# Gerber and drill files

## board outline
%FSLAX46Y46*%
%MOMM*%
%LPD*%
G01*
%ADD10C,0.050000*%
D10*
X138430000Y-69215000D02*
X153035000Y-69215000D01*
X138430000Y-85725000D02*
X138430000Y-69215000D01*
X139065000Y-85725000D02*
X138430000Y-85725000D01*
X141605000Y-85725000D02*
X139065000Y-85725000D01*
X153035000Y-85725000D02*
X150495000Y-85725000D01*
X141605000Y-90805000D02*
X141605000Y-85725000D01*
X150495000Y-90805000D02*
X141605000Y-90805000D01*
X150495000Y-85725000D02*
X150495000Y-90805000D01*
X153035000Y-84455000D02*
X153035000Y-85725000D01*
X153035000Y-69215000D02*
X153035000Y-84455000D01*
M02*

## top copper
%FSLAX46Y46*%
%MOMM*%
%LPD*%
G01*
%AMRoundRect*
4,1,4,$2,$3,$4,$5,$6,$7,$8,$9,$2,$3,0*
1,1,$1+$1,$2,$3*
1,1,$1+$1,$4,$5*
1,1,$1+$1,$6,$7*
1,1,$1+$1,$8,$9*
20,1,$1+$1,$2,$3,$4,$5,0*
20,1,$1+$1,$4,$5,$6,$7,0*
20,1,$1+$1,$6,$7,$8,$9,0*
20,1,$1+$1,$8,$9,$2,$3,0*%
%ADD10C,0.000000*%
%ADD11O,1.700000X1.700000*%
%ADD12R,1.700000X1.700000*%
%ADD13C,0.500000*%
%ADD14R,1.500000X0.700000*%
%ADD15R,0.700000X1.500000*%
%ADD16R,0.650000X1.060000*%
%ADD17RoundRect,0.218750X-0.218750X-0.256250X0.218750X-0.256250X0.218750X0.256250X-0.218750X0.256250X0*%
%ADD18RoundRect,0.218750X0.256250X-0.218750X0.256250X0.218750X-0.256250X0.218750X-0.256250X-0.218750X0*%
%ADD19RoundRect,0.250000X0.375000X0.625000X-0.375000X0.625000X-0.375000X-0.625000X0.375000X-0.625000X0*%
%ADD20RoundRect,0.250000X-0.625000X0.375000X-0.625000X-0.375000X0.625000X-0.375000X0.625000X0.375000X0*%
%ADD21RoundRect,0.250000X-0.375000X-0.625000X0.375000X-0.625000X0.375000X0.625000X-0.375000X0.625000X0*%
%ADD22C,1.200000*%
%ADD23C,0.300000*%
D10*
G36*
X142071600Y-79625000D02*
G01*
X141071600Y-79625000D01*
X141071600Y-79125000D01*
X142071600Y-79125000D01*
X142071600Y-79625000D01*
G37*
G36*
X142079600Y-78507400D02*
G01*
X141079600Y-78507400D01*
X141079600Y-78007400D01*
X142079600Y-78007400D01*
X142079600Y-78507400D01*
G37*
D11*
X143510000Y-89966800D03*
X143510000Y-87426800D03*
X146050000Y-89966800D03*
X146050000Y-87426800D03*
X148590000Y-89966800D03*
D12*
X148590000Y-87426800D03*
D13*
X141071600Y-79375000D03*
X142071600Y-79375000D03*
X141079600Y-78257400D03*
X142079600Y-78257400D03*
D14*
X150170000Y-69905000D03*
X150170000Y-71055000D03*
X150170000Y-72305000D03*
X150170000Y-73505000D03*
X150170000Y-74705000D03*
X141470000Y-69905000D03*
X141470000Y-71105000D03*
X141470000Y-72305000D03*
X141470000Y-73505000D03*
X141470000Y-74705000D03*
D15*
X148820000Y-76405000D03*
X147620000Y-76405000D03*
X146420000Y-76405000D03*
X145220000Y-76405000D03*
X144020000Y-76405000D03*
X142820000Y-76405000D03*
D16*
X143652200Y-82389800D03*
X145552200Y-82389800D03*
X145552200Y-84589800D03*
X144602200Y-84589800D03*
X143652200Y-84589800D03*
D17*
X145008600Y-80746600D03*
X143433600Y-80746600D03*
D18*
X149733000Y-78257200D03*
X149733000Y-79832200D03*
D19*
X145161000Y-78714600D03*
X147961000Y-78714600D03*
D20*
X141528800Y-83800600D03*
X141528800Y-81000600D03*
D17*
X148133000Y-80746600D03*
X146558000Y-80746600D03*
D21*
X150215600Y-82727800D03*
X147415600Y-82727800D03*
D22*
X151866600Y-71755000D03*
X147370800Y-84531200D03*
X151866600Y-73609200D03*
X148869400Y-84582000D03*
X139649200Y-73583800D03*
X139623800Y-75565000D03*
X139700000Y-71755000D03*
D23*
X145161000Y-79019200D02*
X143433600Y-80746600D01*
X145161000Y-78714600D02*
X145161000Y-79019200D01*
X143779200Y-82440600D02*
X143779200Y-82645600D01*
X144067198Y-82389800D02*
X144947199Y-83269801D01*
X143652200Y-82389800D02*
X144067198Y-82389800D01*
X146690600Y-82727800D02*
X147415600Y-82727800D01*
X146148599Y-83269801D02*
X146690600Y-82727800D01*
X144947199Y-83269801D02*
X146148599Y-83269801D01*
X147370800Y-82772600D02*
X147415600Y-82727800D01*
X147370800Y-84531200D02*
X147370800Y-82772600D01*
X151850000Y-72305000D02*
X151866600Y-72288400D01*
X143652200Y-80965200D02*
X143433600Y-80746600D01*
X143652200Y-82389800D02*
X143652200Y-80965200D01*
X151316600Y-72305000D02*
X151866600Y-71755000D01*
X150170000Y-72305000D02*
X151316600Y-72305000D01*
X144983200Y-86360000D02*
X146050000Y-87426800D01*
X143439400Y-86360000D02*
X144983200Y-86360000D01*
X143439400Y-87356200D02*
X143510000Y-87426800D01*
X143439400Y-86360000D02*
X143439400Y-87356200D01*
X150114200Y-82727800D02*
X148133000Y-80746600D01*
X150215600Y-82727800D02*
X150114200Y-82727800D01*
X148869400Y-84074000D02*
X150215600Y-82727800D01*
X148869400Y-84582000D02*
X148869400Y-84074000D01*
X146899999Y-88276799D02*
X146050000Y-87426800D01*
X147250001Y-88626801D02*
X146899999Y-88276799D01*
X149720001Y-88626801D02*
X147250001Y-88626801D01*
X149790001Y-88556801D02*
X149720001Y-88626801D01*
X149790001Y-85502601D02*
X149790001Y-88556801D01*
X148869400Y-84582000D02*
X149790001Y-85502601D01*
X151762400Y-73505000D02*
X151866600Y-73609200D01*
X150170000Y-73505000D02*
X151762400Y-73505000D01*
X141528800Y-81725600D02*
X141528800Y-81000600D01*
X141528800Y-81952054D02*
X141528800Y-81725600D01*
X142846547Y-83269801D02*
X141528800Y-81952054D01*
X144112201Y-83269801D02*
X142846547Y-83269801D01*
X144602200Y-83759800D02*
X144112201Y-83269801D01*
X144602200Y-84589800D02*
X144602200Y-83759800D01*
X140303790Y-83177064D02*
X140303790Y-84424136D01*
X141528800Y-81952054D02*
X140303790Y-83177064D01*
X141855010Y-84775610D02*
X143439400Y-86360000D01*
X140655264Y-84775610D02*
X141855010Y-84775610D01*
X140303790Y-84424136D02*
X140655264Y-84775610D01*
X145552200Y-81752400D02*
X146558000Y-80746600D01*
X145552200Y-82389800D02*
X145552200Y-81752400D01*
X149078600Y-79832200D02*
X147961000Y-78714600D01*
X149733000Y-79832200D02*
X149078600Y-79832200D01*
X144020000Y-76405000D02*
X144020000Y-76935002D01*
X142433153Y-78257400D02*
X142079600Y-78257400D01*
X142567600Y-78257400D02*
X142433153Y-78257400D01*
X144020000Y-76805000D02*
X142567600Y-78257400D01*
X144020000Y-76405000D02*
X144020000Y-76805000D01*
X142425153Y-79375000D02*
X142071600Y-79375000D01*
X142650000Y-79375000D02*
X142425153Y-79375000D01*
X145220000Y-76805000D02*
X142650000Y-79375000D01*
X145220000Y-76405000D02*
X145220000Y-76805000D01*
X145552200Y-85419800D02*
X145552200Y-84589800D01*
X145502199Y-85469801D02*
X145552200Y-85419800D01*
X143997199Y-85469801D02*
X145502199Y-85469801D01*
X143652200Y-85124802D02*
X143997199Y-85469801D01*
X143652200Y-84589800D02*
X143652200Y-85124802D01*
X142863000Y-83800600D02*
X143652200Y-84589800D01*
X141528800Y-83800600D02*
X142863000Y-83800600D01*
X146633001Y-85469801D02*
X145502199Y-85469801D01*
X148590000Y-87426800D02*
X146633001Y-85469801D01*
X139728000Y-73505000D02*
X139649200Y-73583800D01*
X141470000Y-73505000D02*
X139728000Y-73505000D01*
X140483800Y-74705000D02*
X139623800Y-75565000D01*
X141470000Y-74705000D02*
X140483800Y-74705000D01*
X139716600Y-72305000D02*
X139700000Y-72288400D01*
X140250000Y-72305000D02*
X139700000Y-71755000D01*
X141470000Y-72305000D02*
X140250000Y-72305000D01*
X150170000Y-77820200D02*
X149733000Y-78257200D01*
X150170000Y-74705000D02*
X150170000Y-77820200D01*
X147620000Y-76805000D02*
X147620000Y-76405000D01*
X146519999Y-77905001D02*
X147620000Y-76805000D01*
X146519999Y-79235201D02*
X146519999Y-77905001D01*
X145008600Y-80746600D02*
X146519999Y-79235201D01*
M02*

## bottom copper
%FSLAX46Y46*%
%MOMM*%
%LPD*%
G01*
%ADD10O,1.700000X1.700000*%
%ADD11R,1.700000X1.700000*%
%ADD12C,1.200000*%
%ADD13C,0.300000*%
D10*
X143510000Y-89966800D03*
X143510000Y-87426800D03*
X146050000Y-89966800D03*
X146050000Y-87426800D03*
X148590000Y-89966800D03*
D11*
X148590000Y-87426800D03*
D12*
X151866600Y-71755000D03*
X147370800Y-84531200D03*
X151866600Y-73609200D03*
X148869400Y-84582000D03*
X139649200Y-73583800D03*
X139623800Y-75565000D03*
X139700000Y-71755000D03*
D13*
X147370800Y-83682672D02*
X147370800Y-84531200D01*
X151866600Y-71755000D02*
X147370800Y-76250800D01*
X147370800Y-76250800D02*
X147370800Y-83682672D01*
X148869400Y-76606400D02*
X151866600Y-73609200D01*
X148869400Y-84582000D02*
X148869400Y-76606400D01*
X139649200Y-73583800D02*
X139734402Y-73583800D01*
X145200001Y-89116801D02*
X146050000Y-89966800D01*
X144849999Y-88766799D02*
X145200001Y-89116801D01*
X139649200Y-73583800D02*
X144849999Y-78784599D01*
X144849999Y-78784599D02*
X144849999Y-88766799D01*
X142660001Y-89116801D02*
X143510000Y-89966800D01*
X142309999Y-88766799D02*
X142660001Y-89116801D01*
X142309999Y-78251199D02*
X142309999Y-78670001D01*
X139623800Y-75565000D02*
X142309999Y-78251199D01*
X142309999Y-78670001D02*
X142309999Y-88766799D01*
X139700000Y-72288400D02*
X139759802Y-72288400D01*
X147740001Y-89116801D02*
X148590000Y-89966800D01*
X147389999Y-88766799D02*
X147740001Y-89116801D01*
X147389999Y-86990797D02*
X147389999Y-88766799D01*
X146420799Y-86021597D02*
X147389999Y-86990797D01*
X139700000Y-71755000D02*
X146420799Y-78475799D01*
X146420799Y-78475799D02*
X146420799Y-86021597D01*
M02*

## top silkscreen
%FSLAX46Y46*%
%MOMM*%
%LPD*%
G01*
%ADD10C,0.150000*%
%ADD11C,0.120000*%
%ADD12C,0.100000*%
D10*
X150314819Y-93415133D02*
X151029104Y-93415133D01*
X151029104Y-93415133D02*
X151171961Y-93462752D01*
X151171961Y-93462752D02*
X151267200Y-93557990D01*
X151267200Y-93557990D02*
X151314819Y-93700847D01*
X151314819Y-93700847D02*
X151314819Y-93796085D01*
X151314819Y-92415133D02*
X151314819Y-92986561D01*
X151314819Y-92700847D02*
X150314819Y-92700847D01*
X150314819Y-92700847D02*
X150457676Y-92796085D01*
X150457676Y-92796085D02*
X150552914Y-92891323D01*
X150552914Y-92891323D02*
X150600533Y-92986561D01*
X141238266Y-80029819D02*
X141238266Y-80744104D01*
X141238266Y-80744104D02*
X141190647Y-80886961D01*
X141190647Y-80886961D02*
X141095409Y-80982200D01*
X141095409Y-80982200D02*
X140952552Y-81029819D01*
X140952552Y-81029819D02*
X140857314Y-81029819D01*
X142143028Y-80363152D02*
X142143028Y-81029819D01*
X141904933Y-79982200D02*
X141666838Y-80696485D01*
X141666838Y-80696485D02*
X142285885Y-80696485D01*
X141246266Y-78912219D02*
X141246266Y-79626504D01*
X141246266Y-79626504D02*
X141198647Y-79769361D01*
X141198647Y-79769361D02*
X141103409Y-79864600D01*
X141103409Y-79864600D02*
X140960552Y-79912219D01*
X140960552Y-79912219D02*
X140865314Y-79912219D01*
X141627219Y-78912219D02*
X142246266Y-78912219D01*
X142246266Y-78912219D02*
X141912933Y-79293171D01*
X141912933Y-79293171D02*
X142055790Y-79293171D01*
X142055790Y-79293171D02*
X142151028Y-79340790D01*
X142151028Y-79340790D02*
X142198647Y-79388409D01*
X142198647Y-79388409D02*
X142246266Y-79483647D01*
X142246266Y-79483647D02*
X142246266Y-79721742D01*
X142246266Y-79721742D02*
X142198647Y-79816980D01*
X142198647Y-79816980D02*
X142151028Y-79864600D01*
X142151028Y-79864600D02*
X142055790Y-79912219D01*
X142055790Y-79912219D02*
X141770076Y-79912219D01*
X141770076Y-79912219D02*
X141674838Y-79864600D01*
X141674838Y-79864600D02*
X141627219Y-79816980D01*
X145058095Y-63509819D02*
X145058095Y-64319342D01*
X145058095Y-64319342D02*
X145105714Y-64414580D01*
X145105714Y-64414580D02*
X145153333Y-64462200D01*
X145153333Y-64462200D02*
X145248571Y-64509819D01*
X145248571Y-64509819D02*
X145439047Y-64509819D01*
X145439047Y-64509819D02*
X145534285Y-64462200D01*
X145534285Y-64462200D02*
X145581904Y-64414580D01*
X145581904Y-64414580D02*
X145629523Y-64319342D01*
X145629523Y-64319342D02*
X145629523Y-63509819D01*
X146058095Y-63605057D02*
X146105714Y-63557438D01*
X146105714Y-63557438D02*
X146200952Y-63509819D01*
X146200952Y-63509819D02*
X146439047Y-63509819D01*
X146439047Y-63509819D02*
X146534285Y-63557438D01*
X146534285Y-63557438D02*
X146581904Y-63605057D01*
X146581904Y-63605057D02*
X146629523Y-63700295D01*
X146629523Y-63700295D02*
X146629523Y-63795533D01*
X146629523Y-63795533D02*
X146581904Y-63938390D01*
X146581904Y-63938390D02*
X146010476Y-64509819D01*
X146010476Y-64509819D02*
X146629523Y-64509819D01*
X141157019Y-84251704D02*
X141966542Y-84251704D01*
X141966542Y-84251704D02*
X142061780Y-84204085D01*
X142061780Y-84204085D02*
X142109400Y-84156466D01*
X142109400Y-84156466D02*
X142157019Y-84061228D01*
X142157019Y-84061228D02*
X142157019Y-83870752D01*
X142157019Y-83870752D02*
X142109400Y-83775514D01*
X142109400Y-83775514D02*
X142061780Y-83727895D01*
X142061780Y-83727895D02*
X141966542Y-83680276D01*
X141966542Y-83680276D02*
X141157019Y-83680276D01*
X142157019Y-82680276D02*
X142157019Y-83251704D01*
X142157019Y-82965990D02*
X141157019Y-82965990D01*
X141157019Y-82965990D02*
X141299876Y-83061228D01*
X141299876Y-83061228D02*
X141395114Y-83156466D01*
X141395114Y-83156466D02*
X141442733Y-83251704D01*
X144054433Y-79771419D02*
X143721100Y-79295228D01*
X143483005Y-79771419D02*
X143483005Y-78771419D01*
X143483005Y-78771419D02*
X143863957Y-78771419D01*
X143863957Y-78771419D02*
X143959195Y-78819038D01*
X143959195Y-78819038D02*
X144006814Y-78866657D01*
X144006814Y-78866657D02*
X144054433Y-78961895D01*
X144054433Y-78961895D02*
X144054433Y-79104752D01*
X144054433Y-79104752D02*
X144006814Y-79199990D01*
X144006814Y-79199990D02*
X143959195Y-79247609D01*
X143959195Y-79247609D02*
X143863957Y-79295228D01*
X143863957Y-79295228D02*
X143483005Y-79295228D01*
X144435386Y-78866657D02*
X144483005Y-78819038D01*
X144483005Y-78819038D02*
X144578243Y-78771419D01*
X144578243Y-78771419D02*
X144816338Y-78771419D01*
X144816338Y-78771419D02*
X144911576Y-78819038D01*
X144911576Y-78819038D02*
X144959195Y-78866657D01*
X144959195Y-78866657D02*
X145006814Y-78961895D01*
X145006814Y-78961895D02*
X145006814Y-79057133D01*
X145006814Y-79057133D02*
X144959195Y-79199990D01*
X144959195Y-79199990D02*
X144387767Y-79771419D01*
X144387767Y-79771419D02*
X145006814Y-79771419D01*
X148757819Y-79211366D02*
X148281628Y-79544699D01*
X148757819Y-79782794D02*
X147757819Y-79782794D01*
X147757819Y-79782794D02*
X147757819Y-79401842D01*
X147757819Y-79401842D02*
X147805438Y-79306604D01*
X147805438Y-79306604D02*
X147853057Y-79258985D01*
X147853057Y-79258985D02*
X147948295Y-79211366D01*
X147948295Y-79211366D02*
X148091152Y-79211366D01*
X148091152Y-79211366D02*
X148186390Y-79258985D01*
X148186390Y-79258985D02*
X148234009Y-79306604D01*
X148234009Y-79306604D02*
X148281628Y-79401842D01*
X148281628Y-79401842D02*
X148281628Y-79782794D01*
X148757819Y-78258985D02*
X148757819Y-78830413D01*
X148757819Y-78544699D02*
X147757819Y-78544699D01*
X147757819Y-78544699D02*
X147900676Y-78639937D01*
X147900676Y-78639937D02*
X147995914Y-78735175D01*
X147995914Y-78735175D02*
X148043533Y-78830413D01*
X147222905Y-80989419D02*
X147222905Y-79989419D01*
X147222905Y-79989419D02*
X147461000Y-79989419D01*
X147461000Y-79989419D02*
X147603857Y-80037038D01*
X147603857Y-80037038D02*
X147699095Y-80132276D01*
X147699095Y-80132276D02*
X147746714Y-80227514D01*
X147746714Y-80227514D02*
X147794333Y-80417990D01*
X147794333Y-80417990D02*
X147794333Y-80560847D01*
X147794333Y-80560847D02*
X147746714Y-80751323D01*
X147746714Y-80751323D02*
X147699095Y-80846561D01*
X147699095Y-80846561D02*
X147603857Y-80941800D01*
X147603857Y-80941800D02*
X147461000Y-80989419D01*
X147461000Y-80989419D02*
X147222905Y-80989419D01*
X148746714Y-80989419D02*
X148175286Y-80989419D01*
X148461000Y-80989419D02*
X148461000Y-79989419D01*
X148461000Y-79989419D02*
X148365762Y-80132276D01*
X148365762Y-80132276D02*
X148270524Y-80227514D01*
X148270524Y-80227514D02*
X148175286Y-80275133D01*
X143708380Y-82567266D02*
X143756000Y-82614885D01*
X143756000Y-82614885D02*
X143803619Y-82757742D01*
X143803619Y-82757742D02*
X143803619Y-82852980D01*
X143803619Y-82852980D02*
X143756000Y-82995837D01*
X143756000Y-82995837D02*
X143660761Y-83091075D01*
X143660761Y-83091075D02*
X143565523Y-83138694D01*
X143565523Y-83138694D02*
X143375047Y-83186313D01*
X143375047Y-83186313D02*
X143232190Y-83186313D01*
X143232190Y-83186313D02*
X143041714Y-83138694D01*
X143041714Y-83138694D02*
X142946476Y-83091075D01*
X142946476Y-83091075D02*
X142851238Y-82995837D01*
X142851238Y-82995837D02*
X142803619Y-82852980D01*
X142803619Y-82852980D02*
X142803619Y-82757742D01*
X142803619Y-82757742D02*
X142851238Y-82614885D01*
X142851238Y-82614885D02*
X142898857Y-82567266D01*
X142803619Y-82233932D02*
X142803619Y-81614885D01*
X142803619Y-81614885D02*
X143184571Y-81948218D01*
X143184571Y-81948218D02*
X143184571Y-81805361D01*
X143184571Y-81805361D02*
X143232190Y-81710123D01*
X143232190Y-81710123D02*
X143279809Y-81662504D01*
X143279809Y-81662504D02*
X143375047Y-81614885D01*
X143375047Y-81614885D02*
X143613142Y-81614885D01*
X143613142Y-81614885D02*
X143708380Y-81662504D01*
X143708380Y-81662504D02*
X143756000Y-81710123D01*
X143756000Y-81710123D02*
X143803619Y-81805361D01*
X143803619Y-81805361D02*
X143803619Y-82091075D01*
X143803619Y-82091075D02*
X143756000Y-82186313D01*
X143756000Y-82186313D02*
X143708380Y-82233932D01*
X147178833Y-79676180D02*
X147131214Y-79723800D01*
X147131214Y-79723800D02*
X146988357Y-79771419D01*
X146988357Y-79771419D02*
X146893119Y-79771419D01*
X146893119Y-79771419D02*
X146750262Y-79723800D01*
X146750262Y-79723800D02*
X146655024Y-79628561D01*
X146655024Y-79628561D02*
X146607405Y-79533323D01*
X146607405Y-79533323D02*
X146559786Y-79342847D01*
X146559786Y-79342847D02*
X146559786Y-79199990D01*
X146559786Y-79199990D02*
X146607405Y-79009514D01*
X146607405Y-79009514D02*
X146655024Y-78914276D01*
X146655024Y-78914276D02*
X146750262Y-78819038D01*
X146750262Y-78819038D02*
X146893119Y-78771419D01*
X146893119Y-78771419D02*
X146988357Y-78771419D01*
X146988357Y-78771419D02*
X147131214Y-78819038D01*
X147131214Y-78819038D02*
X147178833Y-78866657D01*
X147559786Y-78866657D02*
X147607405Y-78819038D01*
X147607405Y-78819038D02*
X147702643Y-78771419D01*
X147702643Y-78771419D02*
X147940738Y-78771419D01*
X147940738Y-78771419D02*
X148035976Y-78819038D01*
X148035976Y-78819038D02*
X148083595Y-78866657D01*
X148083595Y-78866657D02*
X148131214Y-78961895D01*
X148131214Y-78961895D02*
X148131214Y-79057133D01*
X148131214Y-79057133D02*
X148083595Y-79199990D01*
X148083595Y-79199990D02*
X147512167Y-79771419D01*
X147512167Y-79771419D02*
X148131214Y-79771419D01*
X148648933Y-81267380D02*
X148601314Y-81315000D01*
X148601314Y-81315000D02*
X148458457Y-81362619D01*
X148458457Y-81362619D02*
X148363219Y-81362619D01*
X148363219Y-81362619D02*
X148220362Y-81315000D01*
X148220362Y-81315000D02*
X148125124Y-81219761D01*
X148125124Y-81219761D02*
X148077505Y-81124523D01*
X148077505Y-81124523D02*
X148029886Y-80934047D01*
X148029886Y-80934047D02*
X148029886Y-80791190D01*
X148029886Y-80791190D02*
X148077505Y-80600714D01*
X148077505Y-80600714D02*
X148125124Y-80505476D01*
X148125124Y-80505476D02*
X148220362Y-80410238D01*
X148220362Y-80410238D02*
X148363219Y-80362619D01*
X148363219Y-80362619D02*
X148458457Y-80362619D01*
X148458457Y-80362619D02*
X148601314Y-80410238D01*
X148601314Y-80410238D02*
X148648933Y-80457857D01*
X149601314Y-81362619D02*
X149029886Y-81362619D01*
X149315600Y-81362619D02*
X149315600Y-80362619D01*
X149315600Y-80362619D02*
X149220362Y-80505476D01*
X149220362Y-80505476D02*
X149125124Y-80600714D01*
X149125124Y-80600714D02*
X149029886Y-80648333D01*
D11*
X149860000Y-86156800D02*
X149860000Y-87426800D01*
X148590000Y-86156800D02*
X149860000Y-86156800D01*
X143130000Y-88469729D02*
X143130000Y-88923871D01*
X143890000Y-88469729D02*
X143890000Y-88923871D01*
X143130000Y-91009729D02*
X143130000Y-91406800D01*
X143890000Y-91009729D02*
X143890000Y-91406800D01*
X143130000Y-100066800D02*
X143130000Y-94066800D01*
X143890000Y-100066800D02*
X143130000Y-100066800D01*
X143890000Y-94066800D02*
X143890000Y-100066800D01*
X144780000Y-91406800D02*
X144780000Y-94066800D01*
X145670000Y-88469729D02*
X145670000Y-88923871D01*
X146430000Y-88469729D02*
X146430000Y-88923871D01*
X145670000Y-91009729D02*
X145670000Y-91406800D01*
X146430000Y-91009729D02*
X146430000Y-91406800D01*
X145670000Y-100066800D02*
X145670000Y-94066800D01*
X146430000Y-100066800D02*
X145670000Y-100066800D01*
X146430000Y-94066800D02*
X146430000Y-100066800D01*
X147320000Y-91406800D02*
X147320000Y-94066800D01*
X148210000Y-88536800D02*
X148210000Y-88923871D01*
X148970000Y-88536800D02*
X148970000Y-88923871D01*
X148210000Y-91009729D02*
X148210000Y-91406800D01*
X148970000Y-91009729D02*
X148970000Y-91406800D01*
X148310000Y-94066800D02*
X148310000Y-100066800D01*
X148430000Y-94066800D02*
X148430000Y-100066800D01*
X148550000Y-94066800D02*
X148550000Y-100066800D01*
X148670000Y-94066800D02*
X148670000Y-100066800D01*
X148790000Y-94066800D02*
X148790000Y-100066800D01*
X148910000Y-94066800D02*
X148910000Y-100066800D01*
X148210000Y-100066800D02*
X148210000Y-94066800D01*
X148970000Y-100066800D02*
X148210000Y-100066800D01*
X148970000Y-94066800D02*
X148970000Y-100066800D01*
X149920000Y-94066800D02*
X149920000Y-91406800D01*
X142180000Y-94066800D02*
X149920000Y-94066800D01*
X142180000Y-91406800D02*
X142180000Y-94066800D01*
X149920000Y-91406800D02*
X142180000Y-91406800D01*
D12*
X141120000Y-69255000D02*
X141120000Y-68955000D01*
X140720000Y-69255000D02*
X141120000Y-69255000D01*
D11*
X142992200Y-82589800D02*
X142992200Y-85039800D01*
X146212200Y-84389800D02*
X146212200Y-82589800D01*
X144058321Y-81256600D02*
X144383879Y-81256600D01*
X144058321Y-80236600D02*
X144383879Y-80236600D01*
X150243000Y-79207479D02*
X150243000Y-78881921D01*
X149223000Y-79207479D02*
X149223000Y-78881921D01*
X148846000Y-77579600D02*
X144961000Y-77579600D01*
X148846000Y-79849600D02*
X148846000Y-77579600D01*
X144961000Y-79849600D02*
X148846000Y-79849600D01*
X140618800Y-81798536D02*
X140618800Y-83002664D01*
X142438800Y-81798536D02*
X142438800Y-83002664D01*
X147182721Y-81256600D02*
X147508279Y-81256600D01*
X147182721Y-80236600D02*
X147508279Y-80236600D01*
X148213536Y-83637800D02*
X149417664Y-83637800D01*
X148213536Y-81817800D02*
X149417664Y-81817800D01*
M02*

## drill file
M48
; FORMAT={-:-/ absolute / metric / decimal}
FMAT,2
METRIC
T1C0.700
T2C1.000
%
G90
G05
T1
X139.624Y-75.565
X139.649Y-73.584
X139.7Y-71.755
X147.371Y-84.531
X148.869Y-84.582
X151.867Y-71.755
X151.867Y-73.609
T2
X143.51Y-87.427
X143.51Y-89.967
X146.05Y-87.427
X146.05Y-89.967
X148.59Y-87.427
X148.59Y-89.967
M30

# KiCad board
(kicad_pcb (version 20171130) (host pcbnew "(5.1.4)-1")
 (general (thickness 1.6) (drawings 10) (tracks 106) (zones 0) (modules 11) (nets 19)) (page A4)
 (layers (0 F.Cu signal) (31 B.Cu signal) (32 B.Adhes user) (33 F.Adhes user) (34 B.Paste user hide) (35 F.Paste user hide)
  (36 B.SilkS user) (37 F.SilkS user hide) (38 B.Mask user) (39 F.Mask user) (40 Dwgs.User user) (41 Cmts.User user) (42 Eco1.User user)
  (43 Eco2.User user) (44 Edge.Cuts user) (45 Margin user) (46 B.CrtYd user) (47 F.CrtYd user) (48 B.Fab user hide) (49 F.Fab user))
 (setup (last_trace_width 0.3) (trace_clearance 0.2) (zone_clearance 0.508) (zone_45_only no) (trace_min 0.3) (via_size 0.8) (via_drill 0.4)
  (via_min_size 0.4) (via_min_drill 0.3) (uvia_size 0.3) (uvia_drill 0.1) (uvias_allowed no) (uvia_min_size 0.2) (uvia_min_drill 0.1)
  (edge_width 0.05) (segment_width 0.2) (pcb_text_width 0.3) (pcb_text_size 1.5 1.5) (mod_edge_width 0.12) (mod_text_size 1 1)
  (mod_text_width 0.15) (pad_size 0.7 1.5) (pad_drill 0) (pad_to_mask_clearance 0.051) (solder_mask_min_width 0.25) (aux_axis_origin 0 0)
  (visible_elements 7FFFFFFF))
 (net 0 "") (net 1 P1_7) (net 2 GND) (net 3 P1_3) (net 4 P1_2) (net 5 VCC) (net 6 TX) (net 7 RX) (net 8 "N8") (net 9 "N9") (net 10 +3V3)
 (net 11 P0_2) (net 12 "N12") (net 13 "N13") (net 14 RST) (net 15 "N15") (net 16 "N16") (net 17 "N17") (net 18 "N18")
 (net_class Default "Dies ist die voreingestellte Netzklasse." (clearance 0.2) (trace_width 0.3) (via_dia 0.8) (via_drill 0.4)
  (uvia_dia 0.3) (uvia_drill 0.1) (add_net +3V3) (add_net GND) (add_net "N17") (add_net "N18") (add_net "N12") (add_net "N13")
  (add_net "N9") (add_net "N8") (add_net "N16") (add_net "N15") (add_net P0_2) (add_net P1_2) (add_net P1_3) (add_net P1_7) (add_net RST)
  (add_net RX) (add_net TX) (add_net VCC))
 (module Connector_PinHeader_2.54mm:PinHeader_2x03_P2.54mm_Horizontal (layer F.Cu) (at 148.59 87.4268 270)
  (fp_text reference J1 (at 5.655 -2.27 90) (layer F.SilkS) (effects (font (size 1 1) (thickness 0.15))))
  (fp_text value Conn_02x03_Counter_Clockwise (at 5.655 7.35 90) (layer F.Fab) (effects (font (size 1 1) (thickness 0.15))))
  (fp_line (start -1.27 -1.27) (end 0 -1.27) (layer F.SilkS) (width 0.12))
  (fp_line (start -1.27 0) (end -1.27 -1.27) (layer F.SilkS) (width 0.12))
  (fp_line (start 1.042929 5.46) (end 1.497071 5.46) (layer F.SilkS) (width 0.12))
  (fp_line (start 1.042929 4.7) (end 1.497071 4.7) (layer F.SilkS) (width 0.12))
  (fp_line (start 3.582929 5.46) (end 3.98 5.46) (layer F.SilkS) (width 0.12))
  (fp_line (start 3.582929 4.7) (end 3.98 4.7) (layer F.SilkS) (width 0.12))
  (fp_line (start 12.64 5.46) (end 6.64 5.46) (layer F.SilkS) (width 0.12))
  (fp_line (start 12.64 4.7) (end 12.64 5.46) (layer F.SilkS) (width 0.12))
  (fp_line (start 6.64 4.7) (end 12.64 4.7) (layer F.SilkS) (width 0.12))
  (fp_line (start 3.98 3.81) (end 6.64 3.81) (layer F.SilkS) (width 0.12))
  (fp_line (start 1.042929 2.92) (end 1.497071 2.92) (layer F.SilkS) (width 0.12))
  (fp_line (start 1.042929 2.16) (end 1.497071 2.16) (layer F.SilkS) (width 0.12))
  (fp_line (start 3.582929 2.92) (end 3.98 2.92) (layer F.SilkS) (width 0.12))
  (fp_line (start 3.582929 2.16) (end 3.98 2.16) (layer F.SilkS) (width 0.12))
  (fp_line (start 12.64 2.92) (end 6.64 2.92) (layer F.SilkS) (width 0.12))
  (fp_line (start 12.64 2.16) (end 12.64 2.92) (layer F.SilkS) (width 0.12))
  (fp_line (start 6.64 2.16) (end 12.64 2.16) (layer F.SilkS) (width 0.12))
  (fp_line (start 3.98 1.27) (end 6.64 1.27) (layer F.SilkS) (width 0.12))
  (fp_line (start 1.11 0.38) (end 1.497071 0.38) (layer F.SilkS) (width 0.12))
  (fp_line (start 1.11 -0.38) (end 1.497071 -0.38) (layer F.SilkS) (width 0.12))
  (fp_line (start 3.582929 0.38) (end 3.98 0.38) (layer F.SilkS) (width 0.12))
  (fp_line (start 3.582929 -0.38) (end 3.98 -0.38) (layer F.SilkS) (width 0.12))
  (fp_line (start 6.64 0.28) (end 12.64 0.28) (layer F.SilkS) (width 0.12))
  (fp_line (start 6.64 0.16) (end 12.64 0.16) (layer F.SilkS) (width 0.12))
  (fp_line (start 6.64 0.04) (end 12.64 0.04) (layer F.SilkS) (width 0.12))
  (fp_line (start 6.64 -0.08) (end 12.64 -0.08) (layer F.SilkS) (width 0.12))
  (fp_line (start 6.64 -0.2) (end 12.64 -0.2) (layer F.SilkS) (width 0.12))
  (fp_line (start 6.64 -0.32) (end 12.64 -0.32) (layer F.SilkS) (width 0.12))
  (fp_line (start 12.64 0.38) (end 6.64 0.38) (layer F.SilkS) (width 0.12))
  (fp_line (start 12.64 -0.38) (end 12.64 0.38) (layer F.SilkS) (width 0.12))
  (fp_line (start 6.64 -0.38) (end 12.64 -0.38) (layer F.SilkS) (width 0.12))
  (fp_line (start 6.64 -1.33) (end 3.98 -1.33) (layer F.SilkS) (width 0.12))
  (fp_line (start 6.64 6.41) (end 6.64 -1.33) (layer F.SilkS) (width 0.12))
  (fp_line (start 3.98 6.41) (end 6.64 6.41) (layer F.SilkS) (width 0.12))
  (fp_line (start 3.98 -1.33) (end 3.98 6.41) (layer F.SilkS) (width 0.12))
  (pad 6 thru_hole oval (at 2.54 5.08 270) (size 1.7 1.7) (drill 1) (layers *.Cu) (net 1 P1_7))
  (pad 5 thru_hole oval (at 0 5.08 270) (size 1.7 1.7) (drill 1) (layers *.Cu) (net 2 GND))
  (pad 4 thru_hole oval (at 2.54 2.54 270) (size 1.7 1.7) (drill 1) (layers *.Cu) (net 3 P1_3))
  (pad 3 thru_hole oval (at 0 2.54 270) (size 1.7 1.7) (drill 1) (layers *.Cu) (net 2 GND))
  (pad 2 thru_hole oval (at 2.54 0 270) (size 1.7 1.7) (drill 1) (layers *.Cu) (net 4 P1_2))
  (pad 1 thru_hole rect (at 0 0 270) (size 1.7 1.7) (drill 1) (layers *.Cu) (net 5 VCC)))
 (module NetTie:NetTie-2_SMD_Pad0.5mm (layer F.Cu) (at 141.5716 79.375 180)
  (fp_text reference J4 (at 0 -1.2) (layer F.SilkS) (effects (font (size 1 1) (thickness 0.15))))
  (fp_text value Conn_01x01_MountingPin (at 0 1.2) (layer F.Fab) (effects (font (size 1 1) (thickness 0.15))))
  (fp_poly (pts (xy -0.5 -0.25) (xy 0.5 -0.25) (xy 0.5 0.25) (xy -0.5 0.25)) (layer F.Cu) (width 0))
  (pad 2 smd circle (at 0.5 0 180) (size 0.5 0.5) (layers F.Cu))
  (pad 1 smd circle (at -0.5 0 180) (size 0.5 0.5) (layers F.Cu) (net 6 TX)))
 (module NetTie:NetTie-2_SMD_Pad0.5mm (layer F.Cu) (at 141.5796 78.2574 180)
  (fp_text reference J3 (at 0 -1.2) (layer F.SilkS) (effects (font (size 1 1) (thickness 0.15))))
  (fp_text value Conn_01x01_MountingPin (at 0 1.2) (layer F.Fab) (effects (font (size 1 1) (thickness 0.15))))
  (fp_poly (pts (xy -0.5 -0.25) (xy 0.5 -0.25) (xy 0.5 0.25) (xy -0.5 0.25)) (layer F.Cu) (width 0))
  (pad 2 smd circle (at 0.5 0 180) (size 0.5 0.5) (layers F.Cu))
  (pad 1 smd circle (at -0.5 0 180) (size 0.5 0.5) (layers F.Cu) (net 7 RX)))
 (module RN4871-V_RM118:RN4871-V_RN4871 (layer F.Cu) (at 145.82 73.355)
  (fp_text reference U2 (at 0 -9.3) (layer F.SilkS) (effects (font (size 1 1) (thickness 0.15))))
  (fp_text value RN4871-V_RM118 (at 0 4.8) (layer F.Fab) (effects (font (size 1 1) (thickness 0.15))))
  (fp_line (start -4.7 -4.1) (end -4.7 -4.4) (layer F.SilkS) (width 0.1))
  (fp_line (start -5.1 -4.1) (end -4.7 -4.1) (layer F.SilkS) (width 0.1))
  (pad 16 smd rect (at 4.35 -3.45 90) (size 0.7 1.5) (layers F.Cu) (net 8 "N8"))
  (pad 15 smd rect (at 4.35 -2.3 90) (size 0.7 1.5) (layers F.Cu) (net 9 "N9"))
  (pad 14 smd rect (at 4.35 -1.05 90) (size 0.7 1.5) (layers F.Cu F.Paste F.Mask) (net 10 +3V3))
  (pad 13 smd rect (at 4.35 0.15 90) (size 0.7 1.5) (layers F.Cu F.Paste F.Mask) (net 2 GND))
  (pad 12 smd rect (at 4.35 1.35 90) (size 0.7 1.5) (layers F.Cu F.Paste F.Mask) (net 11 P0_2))
  (pad 1 smd rect (at -4.35 -3.45 90) (size 0.7 1.5) (layers F.Cu) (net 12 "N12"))
  (pad 2 smd rect (at -4.35 -2.25 90) (size 0.7 1.5) (layers F.Cu) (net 2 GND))
  (pad 3 smd rect (at -4.35 -1.05 90) (size 0.7 1.5) (layers F.Cu F.Paste F.Mask) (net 4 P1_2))
  (pad 4 smd rect (at -4.35 0.15 90) (size 0.7 1.5) (layers F.Cu F.Paste F.Mask) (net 3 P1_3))
  (pad 5 smd rect (at -4.35 1.35 90) (size 0.7 1.5) (layers F.Cu F.Paste F.Mask) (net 1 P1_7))
  (pad 11 smd rect (at 3 3.05) (size 0.7 1.5) (layers F.Cu) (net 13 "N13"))
  (pad 10 smd rect (at 1.8 3.05) (size 0.7 1.5) (layers F.Cu F.Paste F.Mask) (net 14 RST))
  (pad 9 smd rect (at 0.6 3.05) (size 0.7 1.5) (layers F.Cu) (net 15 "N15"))
  (pad 8 smd rect (at -0.6 3.05) (size 0.7 1.5) (layers F.Cu F.Paste F.Mask) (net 6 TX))
  (pad 7 smd rect (at -1.8 3.05) (size 0.7 1.5) (layers F.Cu F.Paste F.Mask) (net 7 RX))
  (pad 6 smd rect (at -3 3.05) (size 0.7 1.5) (layers F.Cu) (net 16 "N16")))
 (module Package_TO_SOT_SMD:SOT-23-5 (layer F.Cu) (at 144.6022 83.4898 90)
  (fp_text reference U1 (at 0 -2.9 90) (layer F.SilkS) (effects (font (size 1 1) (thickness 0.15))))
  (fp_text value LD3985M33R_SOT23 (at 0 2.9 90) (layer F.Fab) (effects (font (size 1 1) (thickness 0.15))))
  (fp_line (start 0.9 -1.61) (end -1.55 -1.61) (layer F.SilkS) (width 0.12))
  (fp_line (start -0.9 1.61) (end 0.9 1.61) (layer F.SilkS) (width 0.12))
  (pad 5 smd rect (at 1.1 -0.95 90) (size 1.06 0.65) (layers F.Cu F.Paste F.Mask) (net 10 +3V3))
  (pad 4 smd rect (at 1.1 0.95 90) (size 1.06 0.65) (layers F.Cu F.Paste F.Mask) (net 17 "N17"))
  (pad 3 smd rect (at -1.1 0.95 90) (size 1.06 0.65) (layers F.Cu F.Paste F.Mask) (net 5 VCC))
  (pad 2 smd rect (at -1.1 0 90) (size 1.06 0.65) (layers F.Cu F.Paste F.Mask) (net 2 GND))
  (pad 1 smd rect (at -1.1 -0.95 90) (size 1.06 0.65) (layers F.Cu F.Paste F.Mask) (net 5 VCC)))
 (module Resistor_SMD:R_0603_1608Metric (layer F.Cu) (at 144.2211 80.7466)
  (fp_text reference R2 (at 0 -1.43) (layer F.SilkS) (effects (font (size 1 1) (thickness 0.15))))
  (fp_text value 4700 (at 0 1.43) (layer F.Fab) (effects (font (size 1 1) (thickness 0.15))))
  (fp_line (start -0.162779 0.51) (end 0.162779 0.51) (layer F.SilkS) (width 0.12))
  (fp_line (start -0.162779 -0.51) (end 0.162779 -0.51) (layer F.SilkS) (width 0.12))
  (pad 2 smd roundrect (at 0.7875 0) (size 0.875 0.95) (layers F.Cu F.Paste F.Mask) (roundrect_rratio 0.25) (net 14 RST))
  (pad 1 smd roundrect (at -0.7875 0) (size 0.875 0.95) (layers F.Cu F.Paste F.Mask) (roundrect_rratio 0.25) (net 10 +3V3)))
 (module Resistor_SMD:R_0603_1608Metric (layer F.Cu) (at 149.733 79.0447 90)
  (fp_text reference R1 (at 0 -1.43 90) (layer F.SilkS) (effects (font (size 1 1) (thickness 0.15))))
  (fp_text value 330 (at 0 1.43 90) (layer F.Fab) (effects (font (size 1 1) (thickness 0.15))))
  (fp_line (start -0.162779 0.51) (end 0.162779 0.51) (layer F.SilkS) (width 0.12))
  (fp_line (start -0.162779 -0.51) (end 0.162779 -0.51) (layer F.SilkS) (width 0.12))
  (pad 2 smd roundrect (at 0.7875 0 90) (size 0.875 0.95) (layers F.Cu F.Paste F.Mask) (roundrect_rratio 0.25) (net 11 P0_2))
  (pad 1 smd roundrect (at -0.7875 0 90) (size 0.875 0.95) (layers F.Cu F.Paste F.Mask) (roundrect_rratio 0.25) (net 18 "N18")))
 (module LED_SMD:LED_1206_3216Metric (layer F.Cu) (at 146.561 78.7146 180)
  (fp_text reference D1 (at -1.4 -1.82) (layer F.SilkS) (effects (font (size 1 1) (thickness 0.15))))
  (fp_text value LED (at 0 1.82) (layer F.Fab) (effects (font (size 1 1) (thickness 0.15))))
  (fp_line (start -2.285 1.135) (end 1.6 1.135) (layer F.SilkS) (width 0.12))
  (fp_line (start -2.285 -1.135) (end -2.285 1.135) (layer F.SilkS) (width 0.12))
  (fp_line (start 1.6 -1.135) (end -2.285 -1.135) (layer F.SilkS) (width 0.12))
  (pad 2 smd roundrect (at 1.4 0 180) (size 1.25 1.75) (layers F.Cu F.Paste F.Mask) (roundrect_rratio 0.2) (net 10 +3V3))
  (pad 1 smd roundrect (at -1.4 0 180) (size 1.25 1.75) (layers F.Cu F.Paste F.Mask) (roundrect_rratio 0.2) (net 18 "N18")))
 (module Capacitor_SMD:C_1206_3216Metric (layer F.Cu) (at 141.5288 82.4006 270)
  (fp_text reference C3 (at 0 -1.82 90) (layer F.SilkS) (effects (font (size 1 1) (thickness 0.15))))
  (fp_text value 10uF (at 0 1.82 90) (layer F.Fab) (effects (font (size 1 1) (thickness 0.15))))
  (fp_line (start -0.602064 0.91) (end 0.602064 0.91) (layer F.SilkS) (width 0.12))
  (fp_line (start -0.602064 -0.91) (end 0.602064 -0.91) (layer F.SilkS) (width 0.12))
  (pad 2 smd roundrect (at 1.4 0 270) (size 1.25 1.75) (layers F.Cu F.Paste F.Mask) (roundrect_rratio 0.2) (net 5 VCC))
  (pad 1 smd roundrect (at -1.4 0 270) (size 1.25 1.75) (layers F.Cu F.Paste F.Mask) (roundrect_rratio 0.2) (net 2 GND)))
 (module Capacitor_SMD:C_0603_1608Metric (layer F.Cu) (at 147.3455 80.7466)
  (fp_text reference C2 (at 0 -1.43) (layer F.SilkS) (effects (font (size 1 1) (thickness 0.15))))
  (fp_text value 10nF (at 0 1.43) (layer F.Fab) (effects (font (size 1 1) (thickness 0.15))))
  (fp_line (start -0.162779 0.51) (end 0.162779 0.51) (layer F.SilkS) (width 0.12))
  (fp_line (start -0.162779 -0.51) (end 0.162779 -0.51) (layer F.SilkS) (width 0.12))
  (pad 2 smd roundrect (at 0.7875 0) (size 0.875 0.95) (layers F.Cu F.Paste F.Mask) (roundrect_rratio 0.25) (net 2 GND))
  (pad 1 smd roundrect (at -0.7875 0) (size 0.875 0.95) (layers F.Cu F.Paste F.Mask) (roundrect_rratio 0.25) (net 17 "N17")))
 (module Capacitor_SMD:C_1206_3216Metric (layer F.Cu) (at 148.8156 82.7278)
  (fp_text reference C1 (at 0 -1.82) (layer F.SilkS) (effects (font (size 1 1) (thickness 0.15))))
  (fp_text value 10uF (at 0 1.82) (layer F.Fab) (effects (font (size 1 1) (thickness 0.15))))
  (fp_line (start -0.602064 0.91) (end 0.602064 0.91) (layer F.SilkS) (width 0.12))
  (fp_line (start -0.602064 -0.91) (end 0.602064 -0.91) (layer F.SilkS) (width 0.12))
  (pad 2 smd roundrect (at 1.4 0) (size 1.25 1.75) (layers F.Cu F.Paste F.Mask) (roundrect_rratio 0.2) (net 2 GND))
  (pad 1 smd roundrect (at -1.4 0) (size 1.25 1.75) (layers F.Cu F.Paste F.Mask) (roundrect_rratio 0.2) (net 10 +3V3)))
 (gr_line (start 138.43 69.215) (end 153.035 69.215) (layer Edge.Cuts) (width 0.05))
 (gr_line (start 138.43 85.725) (end 138.43 69.215) (layer Edge.Cuts) (width 0.05))
 (gr_line (start 139.065 85.725) (end 138.43 85.725) (layer Edge.Cuts) (width 0.05))
 (gr_line (start 141.605 85.725) (end 139.065 85.725) (layer Edge.Cuts) (width 0.05))
 (gr_line (start 153.035 85.725) (end 150.495 85.725) (layer Edge.Cuts) (width 0.05))
 (gr_line (start 141.605 90.805) (end 141.605 85.725) (layer Edge.Cuts) (width 0.05))
 (gr_line (start 150.495 90.805) (end 141.605 90.805) (layer Edge.Cuts) (width 0.05))
 (gr_line (start 150.495 85.725) (end 150.495 90.805) (layer Edge.Cuts) (width 0.05))
 (gr_line (start 153.035 84.455) (end 153.035 85.725) (layer Edge.Cuts) (width 0.05))
 (gr_line (start 153.035 69.215) (end 153.035 84.455) (layer Edge.Cuts) (width 0.05))
 (via (at 151.8666 71.755) (size 1.2) (drill 0.7) (layers F.Cu B.Cu) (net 10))
 (via (at 147.3708 84.5312) (size 1.2) (drill 0.7) (layers F.Cu B.Cu) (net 10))
 (segment (start 145.161 79.0192) (end 143.4336 80.7466) (width 0.3) (layer F.Cu) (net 10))
 (segment (start 145.161 78.7146) (end 145.161 79.0192) (width 0.3) (layer F.Cu) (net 10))
 (segment (start 143.7792 82.4406) (end 143.7792 82.6456) (width 0.3) (layer F.Cu) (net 10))
 (segment (start 144.067198 82.3898) (end 144.947199 83.269801) (width 0.3) (layer F.Cu) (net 10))
 (segment (start 143.6522 82.3898) (end 144.067198 82.3898) (width 0.3) (layer F.Cu) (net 10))
 (segment (start 146.6906 82.7278) (end 147.4156 82.7278) (width 0.3) (layer F.Cu) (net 10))
 (segment (start 146.148599 83.269801) (end 146.6906 82.7278) (width 0.3) (layer F.Cu) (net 10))
 (segment (start 144.947199 83.269801) (end 146.148599 83.269801) (width 0.3) (layer F.Cu) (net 10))
 (segment (start 147.3708 82.7726) (end 147.4156 82.7278) (width 0.3) (layer F.Cu) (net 10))
 (segment (start 147.3708 84.5312) (end 147.3708 82.7726) (width 0.3) (layer F.Cu) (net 10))
 (segment (start 151.85 72.305) (end 151.8666 72.2884) (width 0.3) (layer F.Cu) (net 10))
 (segment (start 147.3708 83.682672) (end 147.3708 84.5312) (width 0.3) (layer B.Cu) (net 10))
 (segment (start 143.6522 80.9652) (end 143.4336 80.7466) (width 0.3) (layer F.Cu) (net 10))
 (segment (start 143.6522 82.3898) (end 143.6522 80.9652) (width 0.3) (layer F.Cu) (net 10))
 (segment (start 151.3166 72.305) (end 151.8666 71.755) (width 0.3) (layer F.Cu) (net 10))
 (segment (start 150.17 72.305) (end 151.3166 72.305) (width 0.3) (layer F.Cu) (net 10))
 (segment (start 151.8666 71.755) (end 147.3708 76.2508) (width 0.3) (layer B.Cu) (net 10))
 (segment (start 147.3708 76.2508) (end 147.3708 83.682672) (width 0.3) (layer B.Cu) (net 10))
 (via (at 151.8666 73.6092) (size 1.2) (drill 0.7) (layers F.Cu B.Cu) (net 2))
 (via (at 148.8694 84.582) (size 1.2) (drill 0.7) (layers F.Cu B.Cu) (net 2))
 (segment (start 144.9832 86.36) (end 146.05 87.4268) (width 0.3) (layer F.Cu) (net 2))
 (segment (start 143.4394 86.36) (end 144.9832 86.36) (width 0.3) (layer F.Cu) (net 2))
 (segment (start 143.4394 87.3562) (end 143.51 87.4268) (width 0.3) (layer F.Cu) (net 2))
 (segment (start 143.4394 86.36) (end 143.4394 87.3562) (width 0.3) (layer F.Cu) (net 2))
 (segment (start 150.1142 82.7278) (end 148.133 80.7466) (width 0.3) (layer F.Cu) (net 2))
 (segment (start 150.2156 82.7278) (end 150.1142 82.7278) (width 0.3) (layer F.Cu) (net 2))
 (segment (start 148.8694 84.074) (end 150.2156 82.7278) (width 0.3) (layer F.Cu) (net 2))
 (segment (start 148.8694 84.582) (end 148.8694 84.074) (width 0.3) (layer F.Cu) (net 2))
 (segment (start 146.899999 88.276799) (end 146.05 87.4268) (width 0.3) (layer F.Cu) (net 2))
 (segment (start 147.250001 88.626801) (end 146.899999 88.276799) (width 0.3) (layer F.Cu) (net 2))
 (segment (start 149.720001 88.626801) (end 147.250001 88.626801) (width 0.3) (layer F.Cu) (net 2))
 (segment (start 149.790001 88.556801) (end 149.720001 88.626801) (width 0.3) (layer F.Cu) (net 2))
 (segment (start 149.790001 85.502601) (end 149.790001 88.556801) (width 0.3) (layer F.Cu) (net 2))
 (segment (start 148.8694 84.582) (end 149.790001 85.502601) (width 0.3) (layer F.Cu) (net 2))
 (segment (start 151.7624 73.505) (end 151.8666 73.6092) (width 0.3) (layer F.Cu) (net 2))
 (segment (start 150.17 73.505) (end 151.7624 73.505) (width 0.3) (layer F.Cu) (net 2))
 (segment (start 141.5288 81.7256) (end 141.5288 81.0006) (width 0.3) (layer F.Cu) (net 2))
 (segment (start 141.5288 81.952054) (end 141.5288 81.7256) (width 0.3) (layer F.Cu) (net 2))
 (segment (start 142.846547 83.269801) (end 141.5288 81.952054) (width 0.3) (layer F.Cu) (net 2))
 (segment (start 144.112201 83.269801) (end 142.846547 83.269801) (width 0.3) (layer F.Cu) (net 2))
 (segment (start 144.6022 83.7598) (end 144.112201 83.269801) (width 0.3) (layer F.Cu) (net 2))
 (segment (start 144.6022 84.5898) (end 144.6022 83.7598) (width 0.3) (layer F.Cu) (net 2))
 (segment (start 140.30379 83.177064) (end 140.30379 84.424136) (width 0.3) (layer F.Cu) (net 2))
 (segment (start 141.5288 81.952054) (end 140.30379 83.177064) (width 0.3) (layer F.Cu) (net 2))
 (segment (start 148.8694 76.6064) (end 151.8666 73.6092) (width 0.3) (layer B.Cu) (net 2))
 (segment (start 148.8694 84.582) (end 148.8694 76.6064) (width 0.3) (layer B.Cu) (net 2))
 (segment (start 141.85501 84.77561) (end 143.4394 86.36) (width 0.3) (layer F.Cu) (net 2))
 (segment (start 140.655264 84.77561) (end 141.85501 84.77561) (width 0.3) (layer F.Cu) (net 2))
 (segment (start 140.30379 84.424136) (end 140.655264 84.77561) (width 0.3) (layer F.Cu) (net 2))
 (segment (start 145.5522 81.7524) (end 146.558 80.7466) (width 0.3) (layer F.Cu) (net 17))
 (segment (start 145.5522 82.3898) (end 145.5522 81.7524) (width 0.3) (layer F.Cu) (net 17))
 (segment (start 149.0786 79.8322) (end 147.961 78.7146) (width 0.3) (layer F.Cu) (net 18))
 (segment (start 149.733 79.8322) (end 149.0786 79.8322) (width 0.3) (layer F.Cu) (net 18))
 (segment (start 144.02 76.405) (end 144.02 76.935002) (width 0.3) (layer F.Cu) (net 7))
 (segment (start 142.433153 78.2574) (end 142.0796 78.2574) (width 0.3) (layer F.Cu) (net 7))
 (segment (start 142.5676 78.2574) (end 142.433153 78.2574) (width 0.3) (layer F.Cu) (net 7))
 (segment (start 144.02 76.805) (end 142.5676 78.2574) (width 0.3) (layer F.Cu) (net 7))
 (segment (start 144.02 76.405) (end 144.02 76.805) (width 0.3) (layer F.Cu) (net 7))
 (segment (start 142.425153 79.375) (end 142.0716 79.375) (width 0.3) (layer F.Cu) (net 6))
 (segment (start 142.65 79.375) (end 142.425153 79.375) (width 0.3) (layer F.Cu) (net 6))
 (segment (start 145.22 76.805) (end 142.65 79.375) (width 0.3) (layer F.Cu) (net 6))
 (segment (start 145.22 76.405) (end 145.22 76.805) (width 0.3) (layer F.Cu) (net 6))
 (segment (start 145.5522 85.4198) (end 145.5522 84.5898) (width 0.3) (layer F.Cu) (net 5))
 (segment (start 145.502199 85.469801) (end 145.5522 85.4198) (width 0.3) (layer F.Cu) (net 5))
 (segment (start 143.997199 85.469801) (end 145.502199 85.469801) (width 0.3) (layer F.Cu) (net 5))
 (segment (start 143.6522 85.124802) (end 143.997199 85.469801) (width 0.3) (layer F.Cu) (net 5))
 (segment (start 143.6522 84.5898) (end 143.6522 85.124802) (width 0.3) (layer F.Cu) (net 5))
 (segment (start 142.863 83.8006) (end 143.6522 84.5898) (width 0.3) (layer F.Cu) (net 5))
 (segment (start 141.5288 83.8006) (end 142.863 83.8006) (width 0.3) (layer F.Cu) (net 5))
 (segment (start 146.633001 85.469801) (end 145.502199 85.469801) (width 0.3) (layer F.Cu) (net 5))
 (segment (start 148.59 87.4268) (end 146.633001 85.469801) (width 0.3) (layer F.Cu) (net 5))
 (via (at 139.6492 73.5838) (size 1.2) (drill 0.7) (layers F.Cu B.Cu) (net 3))
 (segment (start 139.6492 73.5838) (end 139.734402 73.5838) (width 0.3) (layer B.Cu) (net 3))
 (segment (start 139.728 73.505) (end 139.6492 73.5838) (width 0.3) (layer F.Cu) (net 3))
 (segment (start 141.47 73.505) (end 139.728 73.505) (width 0.3) (layer F.Cu) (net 3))
 (segment (start 145.200001 89.116801) (end 146.05 89.9668) (width 0.3) (layer B.Cu) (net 3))
 (segment (start 144.849999 88.766799) (end 145.200001 89.116801) (width 0.3) (layer B.Cu) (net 3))
 (segment (start 139.6492 73.5838) (end 144.849999 78.784599) (width 0.3) (layer B.Cu) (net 3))
 (segment (start 144.849999 78.784599) (end 144.849999 88.766799) (width 0.3) (layer B.Cu) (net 3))
 (via (at 139.6238 75.565) (size 1.2) (drill 0.7) (layers F.Cu B.Cu) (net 1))
 (segment (start 142.660001 89.116801) (end 143.51 89.9668) (width 0.3) (layer B.Cu) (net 1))
 (segment (start 142.309999 88.766799) (end 142.660001 89.116801) (width 0.3) (layer B.Cu) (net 1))
 (segment (start 140.4838 74.705) (end 139.6238 75.565) (width 0.3) (layer F.Cu) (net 1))
 (segment (start 141.47 74.705) (end 140.4838 74.705) (width 0.3) (layer F.Cu) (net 1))
 (segment (start 142.309999 78.251199) (end 142.309999 78.670001) (width 0.3) (layer B.Cu) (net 1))
 (segment (start 139.6238 75.565) (end 142.309999 78.251199) (width 0.3) (layer B.Cu) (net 1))
 (segment (start 142.309999 78.670001) (end 142.309999 88.766799) (width 0.3) (layer B.Cu) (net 1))
 (via (at 139.7 71.755) (size 1.2) (drill 0.7) (layers F.Cu B.Cu) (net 4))
 (segment (start 139.7166 72.305) (end 139.7 72.2884) (width 0.3) (layer F.Cu) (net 4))
 (segment (start 139.7 72.2884) (end 139.759802 72.2884) (width 0.3) (layer B.Cu) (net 4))
 (segment (start 140.25 72.305) (end 139.7 71.755) (width 0.3) (layer F.Cu) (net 4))
 (segment (start 141.47 72.305) (end 140.25 72.305) (width 0.3) (layer F.Cu) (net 4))
 (segment (start 147.740001 89.116801) (end 148.59 89.9668) (width 0.3) (layer B.Cu) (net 4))
 (segment (start 147.389999 88.766799) (end 147.740001 89.116801) (width 0.3) (layer B.Cu) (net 4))
 (segment (start 147.389999 86.990797) (end 147.389999 88.766799) (width 0.3) (layer B.Cu) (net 4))
 (segment (start 146.420799 86.021597) (end 147.389999 86.990797) (width 0.3) (layer B.Cu) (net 4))
 (segment (start 139.7 71.755) (end 146.420799 78.475799) (width 0.3) (layer B.Cu) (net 4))
 (segment (start 146.420799 78.475799) (end 146.420799 86.021597) (width 0.3) (layer B.Cu) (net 4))
 (segment (start 150.17 77.8202) (end 149.733 78.2572) (width 0.3) (layer F.Cu) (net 11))
 (segment (start 150.17 74.705) (end 150.17 77.8202) (width 0.3) (layer F.Cu) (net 11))
 (segment (start 147.62 76.805) (end 147.62 76.405) (width 0.3) (layer F.Cu) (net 14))
 (segment (start 146.519999 77.905001) (end 147.62 76.805) (width 0.3) (layer F.Cu) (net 14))
 (segment (start 146.519999 79.235201) (end 146.519999 77.905001) (width 0.3) (layer F.Cu) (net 14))
 (segment (start 145.0086 80.7466) (end 146.519999 79.235201) (width 0.3) (layer F.Cu) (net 14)))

